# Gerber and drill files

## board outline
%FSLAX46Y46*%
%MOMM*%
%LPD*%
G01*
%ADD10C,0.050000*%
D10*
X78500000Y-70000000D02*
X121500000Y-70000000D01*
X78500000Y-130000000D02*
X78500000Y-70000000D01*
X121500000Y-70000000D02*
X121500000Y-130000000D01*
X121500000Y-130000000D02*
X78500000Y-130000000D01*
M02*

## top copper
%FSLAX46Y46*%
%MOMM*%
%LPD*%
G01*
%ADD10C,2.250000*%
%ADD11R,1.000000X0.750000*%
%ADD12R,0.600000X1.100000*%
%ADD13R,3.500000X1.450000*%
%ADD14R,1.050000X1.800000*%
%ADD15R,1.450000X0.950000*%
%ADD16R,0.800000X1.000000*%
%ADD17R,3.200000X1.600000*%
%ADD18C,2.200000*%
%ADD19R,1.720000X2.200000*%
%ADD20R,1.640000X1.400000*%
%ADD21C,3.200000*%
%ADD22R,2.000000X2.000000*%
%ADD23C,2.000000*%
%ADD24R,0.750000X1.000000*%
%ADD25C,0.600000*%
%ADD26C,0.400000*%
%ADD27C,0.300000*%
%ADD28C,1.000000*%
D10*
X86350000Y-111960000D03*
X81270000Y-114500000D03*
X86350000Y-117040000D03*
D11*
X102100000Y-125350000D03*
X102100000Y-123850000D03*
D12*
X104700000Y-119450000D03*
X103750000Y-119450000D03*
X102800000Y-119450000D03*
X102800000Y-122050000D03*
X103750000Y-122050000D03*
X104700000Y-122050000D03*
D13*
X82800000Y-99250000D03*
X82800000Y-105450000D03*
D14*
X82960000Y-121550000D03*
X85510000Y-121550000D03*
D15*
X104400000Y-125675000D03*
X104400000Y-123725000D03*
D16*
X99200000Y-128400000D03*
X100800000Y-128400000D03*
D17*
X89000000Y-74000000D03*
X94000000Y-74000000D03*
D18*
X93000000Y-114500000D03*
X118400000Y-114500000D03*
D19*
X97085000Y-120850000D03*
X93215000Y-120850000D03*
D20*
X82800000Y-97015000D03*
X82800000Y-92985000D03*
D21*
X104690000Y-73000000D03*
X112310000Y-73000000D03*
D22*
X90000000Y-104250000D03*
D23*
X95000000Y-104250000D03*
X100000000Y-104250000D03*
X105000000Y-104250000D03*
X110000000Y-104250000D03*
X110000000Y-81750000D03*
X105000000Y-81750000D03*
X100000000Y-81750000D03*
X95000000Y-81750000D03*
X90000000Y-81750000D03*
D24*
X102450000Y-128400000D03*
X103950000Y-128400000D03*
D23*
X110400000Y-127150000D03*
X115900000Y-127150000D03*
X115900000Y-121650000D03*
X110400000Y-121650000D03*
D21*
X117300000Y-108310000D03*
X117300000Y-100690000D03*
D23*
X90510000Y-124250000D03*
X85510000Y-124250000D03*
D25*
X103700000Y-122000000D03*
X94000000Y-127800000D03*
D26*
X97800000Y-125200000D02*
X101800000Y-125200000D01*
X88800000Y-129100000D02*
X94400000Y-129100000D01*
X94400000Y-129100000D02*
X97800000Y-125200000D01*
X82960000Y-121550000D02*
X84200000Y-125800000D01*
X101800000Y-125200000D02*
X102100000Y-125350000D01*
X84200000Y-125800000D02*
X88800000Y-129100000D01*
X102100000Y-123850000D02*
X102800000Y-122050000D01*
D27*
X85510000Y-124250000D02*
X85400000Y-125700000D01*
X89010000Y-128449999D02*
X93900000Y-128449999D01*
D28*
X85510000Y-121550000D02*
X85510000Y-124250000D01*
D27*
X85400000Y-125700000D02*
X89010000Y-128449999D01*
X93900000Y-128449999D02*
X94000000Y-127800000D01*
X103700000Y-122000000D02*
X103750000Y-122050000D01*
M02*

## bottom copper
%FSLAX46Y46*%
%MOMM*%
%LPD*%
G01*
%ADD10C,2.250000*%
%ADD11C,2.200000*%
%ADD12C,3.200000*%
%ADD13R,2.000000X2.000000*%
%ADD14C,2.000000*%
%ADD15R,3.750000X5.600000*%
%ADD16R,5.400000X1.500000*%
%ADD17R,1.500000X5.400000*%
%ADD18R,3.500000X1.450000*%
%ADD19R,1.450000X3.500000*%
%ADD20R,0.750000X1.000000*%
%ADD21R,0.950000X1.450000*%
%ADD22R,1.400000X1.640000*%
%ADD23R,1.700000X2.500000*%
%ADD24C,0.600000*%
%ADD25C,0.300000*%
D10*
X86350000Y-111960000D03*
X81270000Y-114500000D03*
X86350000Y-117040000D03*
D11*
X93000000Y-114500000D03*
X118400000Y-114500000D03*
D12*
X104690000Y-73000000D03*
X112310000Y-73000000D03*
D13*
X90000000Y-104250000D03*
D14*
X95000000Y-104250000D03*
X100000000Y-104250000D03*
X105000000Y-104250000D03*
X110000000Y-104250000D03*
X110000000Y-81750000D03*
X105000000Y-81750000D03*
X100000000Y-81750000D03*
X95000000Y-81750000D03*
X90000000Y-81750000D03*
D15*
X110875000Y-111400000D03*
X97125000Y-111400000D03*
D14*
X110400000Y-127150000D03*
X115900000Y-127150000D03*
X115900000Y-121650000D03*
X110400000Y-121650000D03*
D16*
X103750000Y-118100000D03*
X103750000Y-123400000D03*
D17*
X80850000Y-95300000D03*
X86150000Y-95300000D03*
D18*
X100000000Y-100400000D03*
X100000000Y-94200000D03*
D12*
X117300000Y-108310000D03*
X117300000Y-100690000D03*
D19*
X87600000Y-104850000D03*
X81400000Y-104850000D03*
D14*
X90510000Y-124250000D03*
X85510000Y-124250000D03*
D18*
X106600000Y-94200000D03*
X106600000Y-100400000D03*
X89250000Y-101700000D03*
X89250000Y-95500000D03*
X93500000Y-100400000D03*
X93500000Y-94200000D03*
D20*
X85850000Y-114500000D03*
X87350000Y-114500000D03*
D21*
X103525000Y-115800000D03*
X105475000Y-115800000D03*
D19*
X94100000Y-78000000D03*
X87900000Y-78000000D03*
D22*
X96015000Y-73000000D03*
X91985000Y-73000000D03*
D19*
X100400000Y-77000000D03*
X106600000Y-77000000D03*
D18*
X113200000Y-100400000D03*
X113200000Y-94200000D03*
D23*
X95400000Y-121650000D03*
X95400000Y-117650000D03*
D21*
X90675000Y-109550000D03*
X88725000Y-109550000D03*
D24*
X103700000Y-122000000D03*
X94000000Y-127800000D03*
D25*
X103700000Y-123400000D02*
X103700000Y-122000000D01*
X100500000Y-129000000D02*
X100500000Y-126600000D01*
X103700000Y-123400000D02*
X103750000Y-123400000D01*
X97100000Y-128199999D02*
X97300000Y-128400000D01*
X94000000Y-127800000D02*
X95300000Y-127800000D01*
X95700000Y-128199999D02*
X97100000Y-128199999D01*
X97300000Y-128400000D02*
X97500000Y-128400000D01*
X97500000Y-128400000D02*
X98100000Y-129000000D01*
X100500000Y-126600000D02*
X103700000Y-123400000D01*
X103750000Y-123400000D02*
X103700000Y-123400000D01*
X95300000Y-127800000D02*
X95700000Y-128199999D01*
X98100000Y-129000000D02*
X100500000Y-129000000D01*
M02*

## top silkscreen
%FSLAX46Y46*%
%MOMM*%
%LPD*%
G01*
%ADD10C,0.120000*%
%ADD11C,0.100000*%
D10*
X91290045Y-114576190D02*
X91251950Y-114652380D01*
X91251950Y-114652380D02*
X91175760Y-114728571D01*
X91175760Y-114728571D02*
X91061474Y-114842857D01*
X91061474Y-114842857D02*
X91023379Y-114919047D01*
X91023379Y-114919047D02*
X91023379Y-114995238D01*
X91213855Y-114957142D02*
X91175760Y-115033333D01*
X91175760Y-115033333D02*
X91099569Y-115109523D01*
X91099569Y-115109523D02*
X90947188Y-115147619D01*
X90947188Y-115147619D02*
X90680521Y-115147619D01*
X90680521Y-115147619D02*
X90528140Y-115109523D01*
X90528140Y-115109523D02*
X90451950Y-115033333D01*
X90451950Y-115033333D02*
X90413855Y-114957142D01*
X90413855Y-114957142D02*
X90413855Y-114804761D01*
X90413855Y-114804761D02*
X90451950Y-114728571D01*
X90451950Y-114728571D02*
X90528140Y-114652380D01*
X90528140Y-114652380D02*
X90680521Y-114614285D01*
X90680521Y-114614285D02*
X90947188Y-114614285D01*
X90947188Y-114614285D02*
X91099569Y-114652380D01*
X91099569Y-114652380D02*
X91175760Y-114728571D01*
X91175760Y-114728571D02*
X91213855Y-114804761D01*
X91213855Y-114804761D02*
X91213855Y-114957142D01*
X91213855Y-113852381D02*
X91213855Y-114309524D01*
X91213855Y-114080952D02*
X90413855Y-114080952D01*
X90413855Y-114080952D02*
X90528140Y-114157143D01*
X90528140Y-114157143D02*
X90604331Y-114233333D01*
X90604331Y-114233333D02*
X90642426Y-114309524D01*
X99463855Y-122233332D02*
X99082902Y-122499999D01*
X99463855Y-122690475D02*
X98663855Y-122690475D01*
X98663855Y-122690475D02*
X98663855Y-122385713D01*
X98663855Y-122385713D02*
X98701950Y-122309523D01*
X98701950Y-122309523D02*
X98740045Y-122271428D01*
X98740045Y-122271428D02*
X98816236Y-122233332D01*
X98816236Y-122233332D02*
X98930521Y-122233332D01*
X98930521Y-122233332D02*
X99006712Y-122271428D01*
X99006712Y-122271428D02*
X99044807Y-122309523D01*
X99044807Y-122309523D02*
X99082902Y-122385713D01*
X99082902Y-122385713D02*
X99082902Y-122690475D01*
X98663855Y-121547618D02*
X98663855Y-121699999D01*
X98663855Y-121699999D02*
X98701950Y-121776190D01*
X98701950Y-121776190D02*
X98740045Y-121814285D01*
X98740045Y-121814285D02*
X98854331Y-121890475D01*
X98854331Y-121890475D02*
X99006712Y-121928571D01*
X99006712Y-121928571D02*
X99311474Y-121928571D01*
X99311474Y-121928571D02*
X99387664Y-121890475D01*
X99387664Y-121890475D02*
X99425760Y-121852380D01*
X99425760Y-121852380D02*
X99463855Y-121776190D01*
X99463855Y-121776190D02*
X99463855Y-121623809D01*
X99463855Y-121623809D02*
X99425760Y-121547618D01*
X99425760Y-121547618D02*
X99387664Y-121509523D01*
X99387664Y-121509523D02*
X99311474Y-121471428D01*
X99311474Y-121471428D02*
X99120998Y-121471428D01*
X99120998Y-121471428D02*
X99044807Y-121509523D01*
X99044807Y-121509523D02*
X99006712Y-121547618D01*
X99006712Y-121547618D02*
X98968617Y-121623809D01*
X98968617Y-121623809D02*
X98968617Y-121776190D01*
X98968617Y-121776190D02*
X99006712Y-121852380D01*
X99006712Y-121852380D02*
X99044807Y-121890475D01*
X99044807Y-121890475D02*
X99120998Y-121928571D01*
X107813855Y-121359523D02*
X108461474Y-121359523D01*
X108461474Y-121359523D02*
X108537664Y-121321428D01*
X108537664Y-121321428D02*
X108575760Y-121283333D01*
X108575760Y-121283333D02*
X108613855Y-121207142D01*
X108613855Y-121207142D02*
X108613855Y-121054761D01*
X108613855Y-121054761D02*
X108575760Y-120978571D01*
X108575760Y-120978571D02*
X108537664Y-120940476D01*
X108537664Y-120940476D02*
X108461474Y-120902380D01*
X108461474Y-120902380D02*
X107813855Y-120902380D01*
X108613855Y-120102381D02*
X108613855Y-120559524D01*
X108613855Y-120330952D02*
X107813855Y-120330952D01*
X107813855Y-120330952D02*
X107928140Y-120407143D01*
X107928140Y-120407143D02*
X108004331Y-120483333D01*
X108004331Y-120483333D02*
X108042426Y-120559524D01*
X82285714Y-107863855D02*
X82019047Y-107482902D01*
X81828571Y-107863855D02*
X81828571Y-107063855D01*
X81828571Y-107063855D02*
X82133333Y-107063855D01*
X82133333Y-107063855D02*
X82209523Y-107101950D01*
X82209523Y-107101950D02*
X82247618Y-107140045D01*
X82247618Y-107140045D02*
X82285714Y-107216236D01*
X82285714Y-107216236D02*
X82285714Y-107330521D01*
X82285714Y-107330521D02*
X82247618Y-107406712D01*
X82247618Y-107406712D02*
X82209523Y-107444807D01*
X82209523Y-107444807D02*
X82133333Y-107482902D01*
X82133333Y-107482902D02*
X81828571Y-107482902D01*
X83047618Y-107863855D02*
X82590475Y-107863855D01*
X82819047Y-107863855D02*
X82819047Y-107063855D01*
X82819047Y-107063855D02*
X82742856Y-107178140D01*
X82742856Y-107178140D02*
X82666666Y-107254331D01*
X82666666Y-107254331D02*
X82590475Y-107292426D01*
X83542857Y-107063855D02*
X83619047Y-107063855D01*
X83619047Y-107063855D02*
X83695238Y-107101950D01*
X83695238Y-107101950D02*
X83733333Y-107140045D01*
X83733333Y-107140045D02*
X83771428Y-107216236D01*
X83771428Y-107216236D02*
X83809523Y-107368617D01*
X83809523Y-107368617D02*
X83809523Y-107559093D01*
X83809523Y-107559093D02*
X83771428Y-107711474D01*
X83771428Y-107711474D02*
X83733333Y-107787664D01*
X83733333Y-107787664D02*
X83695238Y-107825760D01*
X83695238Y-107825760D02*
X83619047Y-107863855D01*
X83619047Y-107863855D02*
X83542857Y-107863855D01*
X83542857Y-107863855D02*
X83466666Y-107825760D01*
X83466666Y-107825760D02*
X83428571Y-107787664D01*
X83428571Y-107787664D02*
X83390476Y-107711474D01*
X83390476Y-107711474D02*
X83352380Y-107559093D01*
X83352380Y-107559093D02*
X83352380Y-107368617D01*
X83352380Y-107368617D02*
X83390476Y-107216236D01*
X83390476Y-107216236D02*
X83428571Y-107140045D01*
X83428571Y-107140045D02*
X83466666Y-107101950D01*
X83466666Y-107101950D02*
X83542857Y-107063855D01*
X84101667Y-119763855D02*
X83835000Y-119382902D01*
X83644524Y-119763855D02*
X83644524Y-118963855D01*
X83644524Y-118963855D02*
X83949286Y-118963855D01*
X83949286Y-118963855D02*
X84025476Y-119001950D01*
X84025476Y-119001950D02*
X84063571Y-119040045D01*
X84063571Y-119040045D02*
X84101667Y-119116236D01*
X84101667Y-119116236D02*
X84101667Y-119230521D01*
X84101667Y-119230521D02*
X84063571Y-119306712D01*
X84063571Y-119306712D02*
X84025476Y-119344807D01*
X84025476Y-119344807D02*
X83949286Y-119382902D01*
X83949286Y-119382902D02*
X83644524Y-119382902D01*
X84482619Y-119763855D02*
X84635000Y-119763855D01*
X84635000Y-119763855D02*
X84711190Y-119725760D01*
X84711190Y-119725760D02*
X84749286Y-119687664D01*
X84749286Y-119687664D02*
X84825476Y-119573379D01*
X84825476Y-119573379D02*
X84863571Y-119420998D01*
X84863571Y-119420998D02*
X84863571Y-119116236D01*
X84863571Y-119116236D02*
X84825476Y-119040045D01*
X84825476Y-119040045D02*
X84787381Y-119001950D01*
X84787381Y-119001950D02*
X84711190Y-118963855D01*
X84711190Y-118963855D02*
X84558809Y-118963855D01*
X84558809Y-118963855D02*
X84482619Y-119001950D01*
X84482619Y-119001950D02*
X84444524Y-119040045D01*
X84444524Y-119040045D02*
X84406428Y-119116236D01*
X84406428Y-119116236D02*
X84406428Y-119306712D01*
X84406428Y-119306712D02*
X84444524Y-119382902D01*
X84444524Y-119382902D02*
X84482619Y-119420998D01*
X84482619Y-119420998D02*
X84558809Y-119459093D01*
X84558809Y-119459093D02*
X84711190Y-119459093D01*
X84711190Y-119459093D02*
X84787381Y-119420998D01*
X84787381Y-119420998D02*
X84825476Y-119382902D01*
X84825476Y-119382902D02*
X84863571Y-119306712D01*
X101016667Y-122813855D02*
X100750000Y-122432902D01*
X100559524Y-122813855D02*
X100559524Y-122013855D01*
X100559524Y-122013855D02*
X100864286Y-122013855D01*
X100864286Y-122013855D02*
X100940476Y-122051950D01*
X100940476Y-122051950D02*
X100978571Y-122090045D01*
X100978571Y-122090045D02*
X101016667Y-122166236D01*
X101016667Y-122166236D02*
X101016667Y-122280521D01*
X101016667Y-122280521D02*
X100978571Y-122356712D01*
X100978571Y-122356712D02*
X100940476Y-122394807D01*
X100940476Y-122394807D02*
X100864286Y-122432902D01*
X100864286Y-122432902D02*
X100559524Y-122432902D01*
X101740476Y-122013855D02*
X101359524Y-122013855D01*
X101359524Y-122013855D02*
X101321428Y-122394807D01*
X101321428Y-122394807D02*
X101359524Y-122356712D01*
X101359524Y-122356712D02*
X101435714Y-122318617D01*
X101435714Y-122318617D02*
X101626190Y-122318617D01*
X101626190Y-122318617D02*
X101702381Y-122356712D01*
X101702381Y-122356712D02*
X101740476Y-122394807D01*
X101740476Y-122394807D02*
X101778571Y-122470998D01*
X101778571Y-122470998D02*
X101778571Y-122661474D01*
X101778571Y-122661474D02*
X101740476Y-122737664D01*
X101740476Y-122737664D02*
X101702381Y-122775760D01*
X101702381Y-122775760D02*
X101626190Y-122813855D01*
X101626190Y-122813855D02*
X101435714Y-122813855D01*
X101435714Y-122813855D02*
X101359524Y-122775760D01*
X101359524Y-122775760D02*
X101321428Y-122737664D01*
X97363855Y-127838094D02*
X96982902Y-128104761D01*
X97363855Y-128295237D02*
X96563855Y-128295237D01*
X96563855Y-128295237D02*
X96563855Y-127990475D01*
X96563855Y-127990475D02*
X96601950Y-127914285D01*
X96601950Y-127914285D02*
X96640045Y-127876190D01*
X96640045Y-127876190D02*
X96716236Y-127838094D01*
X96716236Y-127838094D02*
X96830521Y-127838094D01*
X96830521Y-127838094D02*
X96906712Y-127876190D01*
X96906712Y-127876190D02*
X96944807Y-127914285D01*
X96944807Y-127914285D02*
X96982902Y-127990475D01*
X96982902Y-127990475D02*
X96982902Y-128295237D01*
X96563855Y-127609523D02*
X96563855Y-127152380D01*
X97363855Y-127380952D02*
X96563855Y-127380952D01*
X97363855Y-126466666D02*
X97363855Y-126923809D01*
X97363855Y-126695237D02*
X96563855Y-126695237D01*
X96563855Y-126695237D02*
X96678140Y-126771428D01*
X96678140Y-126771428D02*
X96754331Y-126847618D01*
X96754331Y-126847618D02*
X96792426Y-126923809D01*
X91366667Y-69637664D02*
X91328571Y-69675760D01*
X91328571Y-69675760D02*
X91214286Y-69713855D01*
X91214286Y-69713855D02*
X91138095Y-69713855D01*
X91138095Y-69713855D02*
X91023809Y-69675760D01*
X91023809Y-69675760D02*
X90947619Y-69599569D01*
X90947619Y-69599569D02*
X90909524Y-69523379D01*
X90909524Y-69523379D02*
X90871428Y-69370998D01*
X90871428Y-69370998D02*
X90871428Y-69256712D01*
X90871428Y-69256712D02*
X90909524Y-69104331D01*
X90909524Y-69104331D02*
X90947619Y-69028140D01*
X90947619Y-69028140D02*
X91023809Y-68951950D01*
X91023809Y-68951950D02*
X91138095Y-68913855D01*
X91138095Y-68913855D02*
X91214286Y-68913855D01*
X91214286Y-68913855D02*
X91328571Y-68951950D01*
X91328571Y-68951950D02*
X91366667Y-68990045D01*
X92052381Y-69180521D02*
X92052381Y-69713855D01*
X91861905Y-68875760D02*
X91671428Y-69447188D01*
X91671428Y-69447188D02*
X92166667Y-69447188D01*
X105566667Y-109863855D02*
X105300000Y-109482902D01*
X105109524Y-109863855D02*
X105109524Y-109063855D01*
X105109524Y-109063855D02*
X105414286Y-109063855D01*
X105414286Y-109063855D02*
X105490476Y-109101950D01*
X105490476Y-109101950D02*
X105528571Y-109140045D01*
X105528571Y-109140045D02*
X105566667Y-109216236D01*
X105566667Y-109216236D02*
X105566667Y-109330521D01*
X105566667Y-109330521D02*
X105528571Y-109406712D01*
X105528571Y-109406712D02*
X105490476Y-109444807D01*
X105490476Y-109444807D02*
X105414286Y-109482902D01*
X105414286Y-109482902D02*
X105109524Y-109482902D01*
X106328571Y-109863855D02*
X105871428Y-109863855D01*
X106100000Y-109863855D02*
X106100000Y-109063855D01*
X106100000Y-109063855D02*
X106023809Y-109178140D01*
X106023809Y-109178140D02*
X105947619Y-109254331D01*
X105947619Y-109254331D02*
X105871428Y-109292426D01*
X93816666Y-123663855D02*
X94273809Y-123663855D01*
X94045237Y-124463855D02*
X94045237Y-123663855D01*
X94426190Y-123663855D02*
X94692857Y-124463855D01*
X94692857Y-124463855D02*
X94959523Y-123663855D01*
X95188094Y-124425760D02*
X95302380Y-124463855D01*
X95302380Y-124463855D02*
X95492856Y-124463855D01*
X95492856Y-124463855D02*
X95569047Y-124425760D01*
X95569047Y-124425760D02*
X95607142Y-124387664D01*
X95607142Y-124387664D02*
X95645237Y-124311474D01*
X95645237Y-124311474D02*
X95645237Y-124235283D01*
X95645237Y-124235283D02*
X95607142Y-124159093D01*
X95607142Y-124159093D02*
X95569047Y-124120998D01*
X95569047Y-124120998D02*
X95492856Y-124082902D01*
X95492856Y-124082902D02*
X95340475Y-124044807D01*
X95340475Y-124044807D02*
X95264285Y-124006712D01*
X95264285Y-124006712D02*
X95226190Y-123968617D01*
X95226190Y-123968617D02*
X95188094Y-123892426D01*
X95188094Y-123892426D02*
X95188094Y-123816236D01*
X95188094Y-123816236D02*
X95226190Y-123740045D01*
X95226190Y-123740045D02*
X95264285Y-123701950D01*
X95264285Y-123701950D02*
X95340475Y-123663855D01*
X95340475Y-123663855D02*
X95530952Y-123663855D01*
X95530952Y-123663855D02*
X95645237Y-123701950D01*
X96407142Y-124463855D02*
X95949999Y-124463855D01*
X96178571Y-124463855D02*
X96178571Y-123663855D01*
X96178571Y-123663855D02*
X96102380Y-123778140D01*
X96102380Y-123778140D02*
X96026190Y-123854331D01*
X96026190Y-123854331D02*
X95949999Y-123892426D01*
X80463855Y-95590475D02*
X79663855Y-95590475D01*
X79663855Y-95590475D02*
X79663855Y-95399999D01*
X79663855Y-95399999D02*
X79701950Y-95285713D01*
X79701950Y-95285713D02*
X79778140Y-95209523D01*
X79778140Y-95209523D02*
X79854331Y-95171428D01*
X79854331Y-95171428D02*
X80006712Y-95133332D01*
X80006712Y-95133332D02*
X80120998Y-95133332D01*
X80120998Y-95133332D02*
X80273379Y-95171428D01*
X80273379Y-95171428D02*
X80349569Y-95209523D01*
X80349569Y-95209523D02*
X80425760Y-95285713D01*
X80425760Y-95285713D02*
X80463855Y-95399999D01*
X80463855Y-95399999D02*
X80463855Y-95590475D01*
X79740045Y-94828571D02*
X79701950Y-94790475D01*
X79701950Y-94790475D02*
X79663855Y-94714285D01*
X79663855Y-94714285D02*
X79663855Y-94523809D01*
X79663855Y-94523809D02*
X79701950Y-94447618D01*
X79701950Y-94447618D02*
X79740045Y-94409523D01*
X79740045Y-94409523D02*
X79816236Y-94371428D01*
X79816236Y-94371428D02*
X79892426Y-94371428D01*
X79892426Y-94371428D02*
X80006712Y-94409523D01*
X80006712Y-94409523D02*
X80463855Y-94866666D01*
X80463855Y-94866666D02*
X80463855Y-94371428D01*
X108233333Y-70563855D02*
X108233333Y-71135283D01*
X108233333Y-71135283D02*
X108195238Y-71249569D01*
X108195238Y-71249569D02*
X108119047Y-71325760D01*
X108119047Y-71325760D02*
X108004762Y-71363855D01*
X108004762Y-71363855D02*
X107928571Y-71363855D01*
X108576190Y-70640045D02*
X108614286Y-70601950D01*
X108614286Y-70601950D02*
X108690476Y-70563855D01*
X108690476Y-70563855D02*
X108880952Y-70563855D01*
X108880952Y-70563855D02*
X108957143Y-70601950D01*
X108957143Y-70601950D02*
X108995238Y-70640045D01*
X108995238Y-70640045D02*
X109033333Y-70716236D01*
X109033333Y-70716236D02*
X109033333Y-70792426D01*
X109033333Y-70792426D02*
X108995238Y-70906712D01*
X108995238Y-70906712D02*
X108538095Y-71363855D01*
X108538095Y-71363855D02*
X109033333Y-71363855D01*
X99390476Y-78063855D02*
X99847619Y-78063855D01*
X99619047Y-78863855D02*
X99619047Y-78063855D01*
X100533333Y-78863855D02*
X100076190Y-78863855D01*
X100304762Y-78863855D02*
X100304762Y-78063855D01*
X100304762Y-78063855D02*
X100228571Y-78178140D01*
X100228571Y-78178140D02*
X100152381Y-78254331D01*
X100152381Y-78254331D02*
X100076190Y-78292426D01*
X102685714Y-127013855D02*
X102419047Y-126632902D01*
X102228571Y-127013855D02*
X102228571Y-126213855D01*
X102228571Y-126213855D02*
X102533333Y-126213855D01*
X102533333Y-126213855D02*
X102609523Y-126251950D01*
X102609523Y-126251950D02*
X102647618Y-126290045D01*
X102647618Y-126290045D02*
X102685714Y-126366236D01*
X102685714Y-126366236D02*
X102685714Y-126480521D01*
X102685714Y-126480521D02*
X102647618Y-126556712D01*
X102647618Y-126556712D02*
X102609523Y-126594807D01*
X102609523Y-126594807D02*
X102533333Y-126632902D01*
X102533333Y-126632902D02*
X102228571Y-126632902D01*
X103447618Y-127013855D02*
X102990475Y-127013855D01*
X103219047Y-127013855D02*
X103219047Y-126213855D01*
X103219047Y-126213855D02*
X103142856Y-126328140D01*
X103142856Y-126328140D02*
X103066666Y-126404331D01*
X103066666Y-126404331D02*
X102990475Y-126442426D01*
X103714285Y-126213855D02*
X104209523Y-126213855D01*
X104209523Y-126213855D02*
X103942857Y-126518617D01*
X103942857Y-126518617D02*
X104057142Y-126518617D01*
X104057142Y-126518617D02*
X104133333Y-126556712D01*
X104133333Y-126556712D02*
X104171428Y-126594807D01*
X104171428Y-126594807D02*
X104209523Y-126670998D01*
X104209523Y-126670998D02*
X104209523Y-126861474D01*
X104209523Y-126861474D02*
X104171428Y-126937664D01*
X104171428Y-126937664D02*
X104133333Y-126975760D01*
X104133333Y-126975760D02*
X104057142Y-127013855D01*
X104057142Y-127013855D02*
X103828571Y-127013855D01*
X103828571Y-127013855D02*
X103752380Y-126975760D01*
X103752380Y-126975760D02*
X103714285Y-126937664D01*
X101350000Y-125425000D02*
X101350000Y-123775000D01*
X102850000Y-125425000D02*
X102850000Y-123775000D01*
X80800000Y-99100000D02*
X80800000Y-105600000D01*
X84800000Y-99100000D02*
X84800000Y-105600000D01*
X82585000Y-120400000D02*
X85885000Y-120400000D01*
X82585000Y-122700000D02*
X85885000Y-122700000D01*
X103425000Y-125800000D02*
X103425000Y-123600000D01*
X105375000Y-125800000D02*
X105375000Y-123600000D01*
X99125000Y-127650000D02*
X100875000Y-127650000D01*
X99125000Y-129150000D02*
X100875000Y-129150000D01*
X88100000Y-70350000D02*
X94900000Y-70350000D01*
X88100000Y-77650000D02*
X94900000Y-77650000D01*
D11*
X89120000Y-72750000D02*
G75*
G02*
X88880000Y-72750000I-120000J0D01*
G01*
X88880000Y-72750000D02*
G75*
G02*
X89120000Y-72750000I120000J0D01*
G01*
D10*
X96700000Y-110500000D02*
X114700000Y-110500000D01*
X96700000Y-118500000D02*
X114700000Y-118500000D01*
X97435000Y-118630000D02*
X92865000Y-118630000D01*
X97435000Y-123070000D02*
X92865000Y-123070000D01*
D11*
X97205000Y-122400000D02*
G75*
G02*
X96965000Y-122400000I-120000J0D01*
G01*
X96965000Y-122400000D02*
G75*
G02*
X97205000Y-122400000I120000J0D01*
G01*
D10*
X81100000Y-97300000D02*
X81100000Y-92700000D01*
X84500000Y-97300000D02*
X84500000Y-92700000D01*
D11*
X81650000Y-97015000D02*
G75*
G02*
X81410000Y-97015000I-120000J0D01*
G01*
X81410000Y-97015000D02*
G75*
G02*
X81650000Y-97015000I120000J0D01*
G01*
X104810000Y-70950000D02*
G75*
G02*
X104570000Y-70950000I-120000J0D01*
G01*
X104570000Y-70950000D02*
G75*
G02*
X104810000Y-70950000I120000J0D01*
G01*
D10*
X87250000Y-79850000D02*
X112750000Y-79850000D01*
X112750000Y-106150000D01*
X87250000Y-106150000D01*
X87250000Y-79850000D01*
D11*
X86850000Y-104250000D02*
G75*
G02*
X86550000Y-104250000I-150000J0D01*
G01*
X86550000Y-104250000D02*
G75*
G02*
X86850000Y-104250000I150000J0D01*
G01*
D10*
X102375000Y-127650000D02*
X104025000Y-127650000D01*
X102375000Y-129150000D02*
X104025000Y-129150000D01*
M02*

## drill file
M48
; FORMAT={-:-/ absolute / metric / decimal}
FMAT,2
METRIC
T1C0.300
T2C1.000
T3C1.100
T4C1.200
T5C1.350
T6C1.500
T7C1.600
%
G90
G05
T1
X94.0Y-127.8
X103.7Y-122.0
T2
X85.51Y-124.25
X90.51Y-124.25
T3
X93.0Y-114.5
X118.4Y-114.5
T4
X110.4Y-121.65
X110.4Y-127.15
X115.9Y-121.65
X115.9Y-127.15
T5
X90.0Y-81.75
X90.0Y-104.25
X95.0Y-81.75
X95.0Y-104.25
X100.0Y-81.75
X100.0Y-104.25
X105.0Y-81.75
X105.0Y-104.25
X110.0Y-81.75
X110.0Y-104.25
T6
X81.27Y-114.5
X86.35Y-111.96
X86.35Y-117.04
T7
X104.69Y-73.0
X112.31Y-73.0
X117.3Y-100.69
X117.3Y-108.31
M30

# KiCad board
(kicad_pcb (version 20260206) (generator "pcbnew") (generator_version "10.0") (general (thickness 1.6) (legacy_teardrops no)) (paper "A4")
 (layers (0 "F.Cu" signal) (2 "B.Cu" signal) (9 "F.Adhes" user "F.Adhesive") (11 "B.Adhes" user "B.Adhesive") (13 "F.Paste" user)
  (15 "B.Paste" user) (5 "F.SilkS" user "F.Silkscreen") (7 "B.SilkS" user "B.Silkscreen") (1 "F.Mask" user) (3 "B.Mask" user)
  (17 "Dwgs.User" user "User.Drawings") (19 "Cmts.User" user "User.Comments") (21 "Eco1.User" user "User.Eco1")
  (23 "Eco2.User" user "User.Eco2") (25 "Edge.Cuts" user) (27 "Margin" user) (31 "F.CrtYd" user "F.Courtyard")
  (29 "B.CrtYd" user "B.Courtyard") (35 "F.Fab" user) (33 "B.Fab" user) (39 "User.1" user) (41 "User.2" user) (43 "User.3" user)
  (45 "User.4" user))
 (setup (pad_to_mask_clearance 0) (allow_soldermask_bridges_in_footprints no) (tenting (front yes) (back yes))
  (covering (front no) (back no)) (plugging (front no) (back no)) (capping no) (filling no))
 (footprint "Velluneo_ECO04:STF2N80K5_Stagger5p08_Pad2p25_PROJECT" (layer "F.Cu") (at 86.35 114.5 -90)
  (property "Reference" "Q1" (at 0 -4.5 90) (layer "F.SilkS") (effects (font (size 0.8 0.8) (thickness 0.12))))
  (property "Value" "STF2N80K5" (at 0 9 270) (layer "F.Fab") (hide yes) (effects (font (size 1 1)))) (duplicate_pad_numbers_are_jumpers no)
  (pad "1" thru_hole circle (at -2.54 0 270) (size 2.25 2.25) (drill 1.5) (layers "*.Cu" "*.Mask") (remove_unused_layers no) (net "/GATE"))
  (pad "2" thru_hole circle (at 0 5.08 270) (size 2.25 2.25) (drill 1.5) (layers "*.Cu" "*.Mask") (remove_unused_layers no) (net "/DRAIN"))
  (pad "3" thru_hole circle (at 2.54 0 270) (size 2.25 2.25) (drill 1.5) (layers "*.Cu" "*.Mask") (remove_unused_layers no) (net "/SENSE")))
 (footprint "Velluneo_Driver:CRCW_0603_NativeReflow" (layer "F.Cu") (at 102.1 124.6 90)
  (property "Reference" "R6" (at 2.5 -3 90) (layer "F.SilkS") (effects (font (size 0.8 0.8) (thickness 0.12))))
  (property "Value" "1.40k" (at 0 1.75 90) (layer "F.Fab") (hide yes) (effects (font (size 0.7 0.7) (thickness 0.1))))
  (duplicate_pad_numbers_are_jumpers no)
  (fp_line (start -0.825 -0.75) (end 0.825 -0.75) (stroke (width 0.12) (type default)) (layer "F.SilkS"))
  (fp_line (start -0.825 0.75) (end 0.825 0.75) (stroke (width 0.12) (type default)) (layer "F.SilkS"))
  (pad "1" smd rect (at -0.75 0 90) (size 0.75 1) (layers "F.Cu" "F.Mask" "F.Paste") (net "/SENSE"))
  (pad "2" smd rect (at 0.75 0 90) (size 0.75 1) (layers "F.Cu" "F.Mask" "F.Paste") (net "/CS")))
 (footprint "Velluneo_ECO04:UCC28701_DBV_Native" (layer "F.Cu") (at 103.75 120.75 -90)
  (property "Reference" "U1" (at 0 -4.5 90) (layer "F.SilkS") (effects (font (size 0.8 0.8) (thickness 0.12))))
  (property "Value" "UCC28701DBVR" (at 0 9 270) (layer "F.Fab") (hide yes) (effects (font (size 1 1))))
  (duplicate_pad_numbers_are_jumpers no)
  (pad "1" smd rect (at -1.3 -0.95 270) (size 1.1 0.6) (layers "F.Cu" "F.Mask" "F.Paste") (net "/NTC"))
  (pad "2" smd rect (at -1.3 0 270) (size 1.1 0.6) (layers "F.Cu" "F.Mask" "F.Paste") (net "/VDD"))
  (pad "3" smd rect (at -1.3 0.95 270) (size 1.1 0.6) (layers "F.Cu" "F.Mask" "F.Paste") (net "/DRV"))
  (pad "4" smd rect (at 1.3 0.95 270) (size 1.1 0.6) (layers "F.Cu" "F.Mask" "F.Paste") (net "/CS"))
  (pad "5" smd rect (at 1.3 0 270) (size 1.1 0.6) (layers "F.Cu" "F.Mask" "F.Paste") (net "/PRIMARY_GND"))
  (pad "6" smd rect (at 1.3 -0.95 270) (size 1.1 0.6) (layers "F.Cu" "F.Mask" "F.Paste") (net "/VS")))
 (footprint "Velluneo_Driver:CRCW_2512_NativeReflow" (layer "F.Cu") (at 82.8 102.35 -90)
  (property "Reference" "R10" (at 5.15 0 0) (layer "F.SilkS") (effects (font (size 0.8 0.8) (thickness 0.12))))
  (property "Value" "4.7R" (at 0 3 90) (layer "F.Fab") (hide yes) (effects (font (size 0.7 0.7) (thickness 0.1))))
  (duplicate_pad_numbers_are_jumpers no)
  (fp_line (start -3.25 2) (end 3.25 2) (stroke (width 0.12) (type default)) (layer "F.SilkS"))
  (fp_line (start -3.25 -2) (end 3.25 -2) (stroke (width 0.12) (type default)) (layer "F.SilkS"))
  (pad "1" smd rect (at -3.1 0 270) (size 1.45 3.5) (layers "F.Cu" "F.Mask" "F.Paste") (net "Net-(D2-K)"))
  (pad "2" smd rect (at 3.1 0 270) (size 1.45 3.5) (layers "F.Cu" "F.Mask" "F.Paste") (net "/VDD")))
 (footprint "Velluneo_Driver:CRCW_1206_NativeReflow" (layer "F.Cu") (at 84.235 121.55)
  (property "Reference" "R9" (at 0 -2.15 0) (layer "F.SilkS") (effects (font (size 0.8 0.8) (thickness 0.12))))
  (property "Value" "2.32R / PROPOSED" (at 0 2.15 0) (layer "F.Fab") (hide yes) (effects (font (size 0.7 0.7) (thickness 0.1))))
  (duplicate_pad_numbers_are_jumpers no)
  (fp_line (start -1.65 -1.15) (end 1.65 -1.15) (stroke (width 0.12) (type default)) (layer "F.SilkS"))
  (fp_line (start -1.65 1.15) (end 1.65 1.15) (stroke (width 0.12) (type default)) (layer "F.SilkS"))
  (pad "1" smd rect (at -1.275 0) (size 1.05 1.8) (layers "F.Cu" "F.Mask" "F.Paste") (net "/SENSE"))
  (pad "2" smd rect (at 1.275 0) (size 1.05 1.8) (layers "F.Cu" "F.Mask" "F.Paste") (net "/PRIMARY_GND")))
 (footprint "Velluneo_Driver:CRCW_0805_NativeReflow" (layer "F.Cu") (at 104.4 124.7 90)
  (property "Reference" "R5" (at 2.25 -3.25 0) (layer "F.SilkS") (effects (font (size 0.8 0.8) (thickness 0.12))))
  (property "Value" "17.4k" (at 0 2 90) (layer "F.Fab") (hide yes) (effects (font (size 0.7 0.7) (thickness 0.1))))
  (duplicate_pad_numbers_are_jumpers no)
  (fp_line (start -1.1 -0.975) (end 1.1 -0.975) (stroke (width 0.12) (type default)) (layer "F.SilkS"))
  (fp_line (start -1.1 0.975) (end 1.1 0.975) (stroke (width 0.12) (type default)) (layer "F.SilkS"))
  (pad "1" smd rect (at -0.975 0 90) (size 0.95 1.45) (layers "F.Cu" "F.Mask" "F.Paste") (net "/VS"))
  (pad "2" smd rect (at 0.975 0 90) (size 0.95 1.45) (layers "F.Cu" "F.Mask" "F.Paste") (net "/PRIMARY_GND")))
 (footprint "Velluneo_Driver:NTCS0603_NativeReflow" (layer "F.Cu") (at 100 128.4)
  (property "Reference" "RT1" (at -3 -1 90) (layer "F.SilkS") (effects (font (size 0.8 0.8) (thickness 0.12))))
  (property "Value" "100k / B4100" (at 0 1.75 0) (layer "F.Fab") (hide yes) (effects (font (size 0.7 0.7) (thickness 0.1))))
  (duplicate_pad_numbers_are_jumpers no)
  (fp_line (start -0.875 -0.75) (end 0.875 -0.75) (stroke (width 0.12) (type default)) (layer "F.SilkS"))
  (fp_line (start -0.875 0.75) (end 0.875 0.75) (stroke (width 0.12) (type default)) (layer "F.SilkS"))
  (pad "1" smd rect (at -0.8 0) (size 0.8 1) (layers "F.Cu" "F.Mask" "F.Paste") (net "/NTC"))
  (pad "2" smd rect (at 0.8 0) (size 0.8 1) (layers "F.Cu" "F.Mask" "F.Paste") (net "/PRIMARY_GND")))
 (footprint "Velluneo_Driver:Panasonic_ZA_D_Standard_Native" (layer "F.Cu") (at 91.5 74)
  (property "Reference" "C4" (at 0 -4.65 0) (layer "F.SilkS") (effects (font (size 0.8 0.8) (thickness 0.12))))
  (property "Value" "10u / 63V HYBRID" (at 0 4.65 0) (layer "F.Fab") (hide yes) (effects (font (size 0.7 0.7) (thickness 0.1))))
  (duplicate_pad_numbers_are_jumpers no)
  (fp_line (start -3.4 -3.65) (end 3.4 -3.65) (stroke (width 0.12) (type default)) (layer "F.SilkS"))
  (fp_line (start -3.4 3.65) (end 3.4 3.65) (stroke (width 0.12) (type default)) (layer "F.SilkS"))
  (fp_circle (center -2.5 -1.25) (end -2.38 -1.25) (stroke (width 0.1) (type default)) (fill no) (layer "F.SilkS"))
  (pad "1" smd rect (at -2.5 0) (size 3.2 1.6) (layers "F.Cu" "F.Mask" "F.Paste") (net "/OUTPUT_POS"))
  (pad "2" smd rect (at 2.5 0) (size 3.2 1.6) (layers "F.Cu" "F.Mask" "F.Paste") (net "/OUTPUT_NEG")))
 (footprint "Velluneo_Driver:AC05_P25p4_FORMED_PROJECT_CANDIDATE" (layer "F.Cu") (at 105.7 114.5)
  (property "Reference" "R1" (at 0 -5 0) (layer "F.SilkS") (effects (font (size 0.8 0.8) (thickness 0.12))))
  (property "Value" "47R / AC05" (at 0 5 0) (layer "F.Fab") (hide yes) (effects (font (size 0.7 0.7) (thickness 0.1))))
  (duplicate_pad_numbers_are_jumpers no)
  (fp_line (start -9 -4) (end 9 -4) (stroke (width 0.12) (type default)) (layer "F.SilkS"))
  (fp_line (start -9 4) (end 9 4) (stroke (width 0.12) (type default)) (layer "F.SilkS"))
  (pad "1" thru_hole circle (at -12.7 0) (size 2.2 2.2) (drill 1.1) (layers "*.Cu" "*.Mask") (remove_unused_layers no) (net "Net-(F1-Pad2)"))
  (pad "2" thru_hole circle (at 12.7 0) (size 2.2 2.2) (drill 1.1) (layers "*.Cu" "*.Mask") (remove_unused_layers no)
   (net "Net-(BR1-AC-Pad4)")))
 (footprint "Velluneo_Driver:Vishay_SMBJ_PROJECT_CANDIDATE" (layer "F.Cu") (at 95.15 120.85 180)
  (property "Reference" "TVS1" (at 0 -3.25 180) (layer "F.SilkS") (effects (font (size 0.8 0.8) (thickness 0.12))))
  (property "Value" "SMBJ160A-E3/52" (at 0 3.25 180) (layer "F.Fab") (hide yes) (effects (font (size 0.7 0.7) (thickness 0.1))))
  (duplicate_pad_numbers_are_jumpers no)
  (fp_line (start -2.285 2.22) (end 2.285 2.22) (stroke (width 0.12) (type default)) (layer "F.SilkS"))
  (fp_line (start -2.285 -2.22) (end 2.285 -2.22) (stroke (width 0.12) (type default)) (layer "F.SilkS"))
  (fp_circle (center -1.935 -1.55) (end -1.815 -1.55) (stroke (width 0.1) (type default)) (fill no) (layer "F.SilkS"))
  (pad "1" smd rect (at -1.935 0 180) (size 1.72 2.2) (layers "F.Cu" "F.Mask" "F.Paste") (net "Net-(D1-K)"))
  (pad "2" smd rect (at 1.935 0 180) (size 1.72 2.2) (layers "F.Cu" "F.Mask" "F.Paste") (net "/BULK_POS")))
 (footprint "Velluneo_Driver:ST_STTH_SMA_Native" (layer "F.Cu") (at 82.8 95 90)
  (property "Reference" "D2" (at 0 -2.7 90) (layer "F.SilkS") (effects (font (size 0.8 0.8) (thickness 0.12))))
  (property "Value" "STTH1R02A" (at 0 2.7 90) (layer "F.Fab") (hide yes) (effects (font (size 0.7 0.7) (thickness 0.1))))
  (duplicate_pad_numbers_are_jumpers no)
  (fp_line (start -2.3 -1.7) (end 2.3 -1.7) (stroke (width 0.12) (type default)) (layer "F.SilkS"))
  (fp_line (start -2.3 1.7) (end 2.3 1.7) (stroke (width 0.12) (type default)) (layer "F.SilkS"))
  (fp_circle (center -2.015 -1.27) (end -1.895 -1.27) (stroke (width 0.1) (type default)) (fill no) (layer "F.SilkS"))
  (pad "1" smd rect (at -2.015 0 90) (size 1.4 1.64) (layers "F.Cu" "F.Mask" "F.Paste") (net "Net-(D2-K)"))
  (pad "2" smd rect (at 2.015 0 90) (size 1.4 1.64) (layers "F.Cu" "F.Mask" "F.Paste") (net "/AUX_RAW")))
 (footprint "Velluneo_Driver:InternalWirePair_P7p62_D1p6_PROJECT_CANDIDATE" (layer "F.Cu") (at 108.5 73)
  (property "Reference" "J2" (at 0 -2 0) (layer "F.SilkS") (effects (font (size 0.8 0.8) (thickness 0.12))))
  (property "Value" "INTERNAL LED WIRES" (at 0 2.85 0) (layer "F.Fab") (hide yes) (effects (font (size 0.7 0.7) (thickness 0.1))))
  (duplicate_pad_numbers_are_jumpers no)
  (fp_circle (center -3.81 -2.05) (end -3.69 -2.05) (stroke (width 0.1) (type default)) (fill no) (layer "F.SilkS"))
  (pad "1" thru_hole circle (at -3.81 0) (size 3.2 3.2) (drill 1.6) (layers "*.Cu" "*.Mask") (remove_unused_layers no) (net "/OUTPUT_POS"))
  (pad "2" thru_hole circle (at 3.81 0) (size 3.2 3.2) (drill 1.6) (layers "*.Cu" "*.Mask") (remove_unused_layers no) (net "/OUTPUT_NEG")))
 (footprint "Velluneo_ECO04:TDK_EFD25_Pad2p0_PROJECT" (layer "F.Cu") (at 100 93)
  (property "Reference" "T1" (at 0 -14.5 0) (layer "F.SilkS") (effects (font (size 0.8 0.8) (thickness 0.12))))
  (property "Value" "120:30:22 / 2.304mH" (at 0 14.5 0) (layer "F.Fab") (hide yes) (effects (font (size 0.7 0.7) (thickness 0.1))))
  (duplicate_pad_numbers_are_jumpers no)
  (fp_rect (start -12.75 -13.15) (end 12.75 13.15) (stroke (width 0.12) (type default)) (fill no) (layer "F.SilkS"))
  (fp_circle (center -13.3 11.25) (end -13.15 11.25) (stroke (width 0.1) (type default)) (fill no) (layer "F.SilkS"))
  (pad "1" thru_hole rect (at -10 11.25) (size 2 2) (drill 1.35) (layers "*.Cu" "*.Mask") (remove_unused_layers no) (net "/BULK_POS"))
  (pad "2" thru_hole circle (at -5 11.25) (size 2 2) (drill 1.35) (layers "*.Cu" "*.Mask") (remove_unused_layers no) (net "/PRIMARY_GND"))
  (pad "3" thru_hole circle (at 0 11.25) (size 2 2) (drill 1.35) (layers "*.Cu" "*.Mask") (remove_unused_layers no)
   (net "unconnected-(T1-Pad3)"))
  (pad "4" thru_hole circle (at 5 11.25) (size 2 2) (drill 1.35) (layers "*.Cu" "*.Mask") (remove_unused_layers no) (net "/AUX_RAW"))
  (pad "5" thru_hole circle (at 10 11.25) (size 2 2) (drill 1.35) (layers "*.Cu" "*.Mask") (remove_unused_layers no) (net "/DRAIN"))
  (pad "6" thru_hole circle (at 10 -11.25) (size 2 2) (drill 1.35) (layers "*.Cu" "*.Mask") (remove_unused_layers no) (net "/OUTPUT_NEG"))
  (pad "7" thru_hole circle (at 5 -11.25) (size 2 2) (drill 1.35) (layers "*.Cu" "*.Mask") (remove_unused_layers no)
   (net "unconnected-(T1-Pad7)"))
  (pad "8" thru_hole circle (at 0 -11.25) (size 2 2) (drill 1.35) (layers "*.Cu" "*.Mask") (remove_unused_layers no)
   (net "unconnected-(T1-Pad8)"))
  (pad "9" thru_hole circle (at -5 -11.25) (size 2 2) (drill 1.35) (layers "*.Cu" "*.Mask") (remove_unused_layers no)
   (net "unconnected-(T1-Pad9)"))
  (pad "10" thru_hole circle (at -10 -11.25) (size 2 2) (drill 1.35) (layers "*.Cu" "*.Mask") (remove_unused_layers no)
   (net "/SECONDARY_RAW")))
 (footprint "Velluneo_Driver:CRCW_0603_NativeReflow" (layer "F.Cu") (at 103.2 128.4)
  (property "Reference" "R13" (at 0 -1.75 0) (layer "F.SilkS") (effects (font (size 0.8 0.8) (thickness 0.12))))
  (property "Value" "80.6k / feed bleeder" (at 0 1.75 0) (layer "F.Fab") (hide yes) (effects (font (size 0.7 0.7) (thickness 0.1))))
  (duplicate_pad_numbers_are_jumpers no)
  (fp_line (start -0.825 -0.75) (end 0.825 -0.75) (stroke (width 0.12) (type default)) (layer "F.SilkS"))
  (fp_line (start -0.825 0.75) (end 0.825 0.75) (stroke (width 0.12) (type default)) (layer "F.SilkS"))
  (pad "1" smd rect (at -0.75 0) (size 0.75 1) (layers "F.Cu" "F.Mask" "F.Paste") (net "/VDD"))
  (pad "2" smd rect (at 0.75 0) (size 0.75 1) (layers "F.Cu" "F.Mask" "F.Paste") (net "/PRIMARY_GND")))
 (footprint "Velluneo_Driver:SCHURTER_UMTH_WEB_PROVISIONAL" (layer "B.Cu") (at 104 111.4 180)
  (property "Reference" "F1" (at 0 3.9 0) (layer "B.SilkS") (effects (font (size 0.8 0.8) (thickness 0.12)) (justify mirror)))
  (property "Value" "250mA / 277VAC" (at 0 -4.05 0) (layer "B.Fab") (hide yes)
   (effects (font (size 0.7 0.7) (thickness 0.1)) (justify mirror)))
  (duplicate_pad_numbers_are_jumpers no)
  (pad "1" smd rect (at -6.875 0 180) (size 3.75 5.6) (layers "B.Cu" "B.Mask" "B.Paste") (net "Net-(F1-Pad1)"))
  (pad "2" smd rect (at 6.875 0 180) (size 3.75 5.6) (layers "B.Cu" "B.Mask" "B.Paste") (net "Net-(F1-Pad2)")))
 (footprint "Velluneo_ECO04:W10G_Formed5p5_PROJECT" (layer "B.Cu") (at 113.15 124.4)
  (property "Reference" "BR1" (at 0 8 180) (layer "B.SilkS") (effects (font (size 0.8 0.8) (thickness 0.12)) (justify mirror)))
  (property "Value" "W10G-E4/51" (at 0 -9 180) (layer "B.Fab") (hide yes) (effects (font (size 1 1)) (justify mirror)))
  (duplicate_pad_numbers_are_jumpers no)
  (pad "1" thru_hole circle (at -2.75 2.75) (size 2 2) (drill 1.2) (layers "*.Cu" "*.Mask") (remove_unused_layers no) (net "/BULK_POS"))
  (pad "2" thru_hole circle (at 2.75 2.75) (size 2 2) (drill 1.2) (layers "*.Cu" "*.Mask") (remove_unused_layers no)
   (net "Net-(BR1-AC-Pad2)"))
  (pad "3" thru_hole circle (at 2.75 -2.75) (size 2 2) (drill 1.2) (layers "*.Cu" "*.Mask") (remove_unused_layers no) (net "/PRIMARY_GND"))
  (pad "4" thru_hole circle (at -2.75 -2.75) (size 2 2) (drill 1.2) (layers "*.Cu" "*.Mask") (remove_unused_layers no)
   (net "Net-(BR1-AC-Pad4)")))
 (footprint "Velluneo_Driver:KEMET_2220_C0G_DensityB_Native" (layer "B.Cu") (at 103.75 120.75 -90)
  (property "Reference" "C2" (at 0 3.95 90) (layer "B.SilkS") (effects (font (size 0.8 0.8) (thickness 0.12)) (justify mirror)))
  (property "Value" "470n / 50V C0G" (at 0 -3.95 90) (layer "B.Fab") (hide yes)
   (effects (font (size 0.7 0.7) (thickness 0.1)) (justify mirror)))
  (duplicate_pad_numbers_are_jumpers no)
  (pad "1" smd rect (at -2.65 0 270) (size 1.5 5.4) (layers "B.Cu" "B.Mask" "B.Paste") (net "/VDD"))
  (pad "2" smd rect (at 2.65 0 270) (size 1.5 5.4) (layers "B.Cu" "B.Mask" "B.Paste") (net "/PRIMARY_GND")))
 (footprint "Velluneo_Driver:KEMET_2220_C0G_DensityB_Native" (layer "B.Cu") (at 83.5 95.3)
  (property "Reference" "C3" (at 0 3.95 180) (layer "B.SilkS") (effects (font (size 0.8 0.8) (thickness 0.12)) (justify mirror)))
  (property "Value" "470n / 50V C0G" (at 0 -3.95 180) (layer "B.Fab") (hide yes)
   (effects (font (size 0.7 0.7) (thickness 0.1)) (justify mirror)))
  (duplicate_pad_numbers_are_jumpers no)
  (pad "1" smd rect (at -2.65 0) (size 1.5 5.4) (layers "B.Cu" "B.Mask" "B.Paste") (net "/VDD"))
  (pad "2" smd rect (at 2.65 0) (size 1.5 5.4) (layers "B.Cu" "B.Mask" "B.Paste") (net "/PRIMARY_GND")))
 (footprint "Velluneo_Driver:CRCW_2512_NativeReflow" (layer "B.Cu") (at 100 97.3 90)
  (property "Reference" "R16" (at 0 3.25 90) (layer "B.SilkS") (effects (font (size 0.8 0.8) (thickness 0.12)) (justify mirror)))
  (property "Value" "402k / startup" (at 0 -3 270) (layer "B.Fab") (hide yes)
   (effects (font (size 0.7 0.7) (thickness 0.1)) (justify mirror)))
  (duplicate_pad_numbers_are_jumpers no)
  (pad "1" smd rect (at -3.1 0 90) (size 1.45 3.5) (layers "B.Cu" "B.Mask" "B.Paste") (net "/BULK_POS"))
  (pad "2" smd rect (at 3.1 0 90) (size 1.45 3.5) (layers "B.Cu" "B.Mask" "B.Paste") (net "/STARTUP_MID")))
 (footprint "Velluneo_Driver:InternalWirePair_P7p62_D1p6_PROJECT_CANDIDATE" (layer "B.Cu") (at 117.3 104.5 90)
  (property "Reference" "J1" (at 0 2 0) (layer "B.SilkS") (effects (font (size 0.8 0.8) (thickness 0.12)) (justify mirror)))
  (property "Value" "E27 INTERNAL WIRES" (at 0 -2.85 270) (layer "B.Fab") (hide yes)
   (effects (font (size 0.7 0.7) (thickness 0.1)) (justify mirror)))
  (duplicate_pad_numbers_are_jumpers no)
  (pad "1" thru_hole circle (at -3.81 0 90) (size 3.2 3.2) (drill 1.6) (layers "*.Cu" "*.Mask") (remove_unused_layers no)
   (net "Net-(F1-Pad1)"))
  (pad "2" thru_hole circle (at 3.81 0 90) (size 3.2 3.2) (drill 1.6) (layers "*.Cu" "*.Mask") (remove_unused_layers no)
   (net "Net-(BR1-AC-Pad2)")))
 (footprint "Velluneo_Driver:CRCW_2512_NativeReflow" (layer "B.Cu") (at 84.5 104.85 180)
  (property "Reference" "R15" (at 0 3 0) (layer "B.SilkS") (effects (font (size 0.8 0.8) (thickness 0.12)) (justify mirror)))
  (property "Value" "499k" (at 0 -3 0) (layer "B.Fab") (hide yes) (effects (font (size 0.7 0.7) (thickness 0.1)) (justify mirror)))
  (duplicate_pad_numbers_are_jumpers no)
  (pad "1" smd rect (at -3.1 0 180) (size 1.45 3.5) (layers "B.Cu" "B.Mask" "B.Paste") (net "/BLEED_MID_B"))
  (pad "2" smd rect (at 3.1 0 180) (size 1.45 3.5) (layers "B.Cu" "B.Mask" "B.Paste") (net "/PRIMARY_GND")))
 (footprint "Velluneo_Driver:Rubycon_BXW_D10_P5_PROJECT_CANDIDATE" (layer "B.Cu") (at 88.01 124.25 180)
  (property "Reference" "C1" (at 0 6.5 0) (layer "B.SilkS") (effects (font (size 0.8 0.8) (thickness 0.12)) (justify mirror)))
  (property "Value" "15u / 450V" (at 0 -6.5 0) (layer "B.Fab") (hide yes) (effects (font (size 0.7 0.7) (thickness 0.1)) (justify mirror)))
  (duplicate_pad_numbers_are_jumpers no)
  (pad "1" thru_hole circle (at -2.5 0 180) (size 2 2) (drill 1) (layers "*.Cu" "*.Mask") (remove_unused_layers no) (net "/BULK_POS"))
  (pad "2" thru_hole circle (at 2.5 0 180) (size 2 2) (drill 1) (layers "*.Cu" "*.Mask") (remove_unused_layers no) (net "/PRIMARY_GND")))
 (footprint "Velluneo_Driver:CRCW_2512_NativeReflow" (layer "B.Cu") (at 106.6 97.3 -90)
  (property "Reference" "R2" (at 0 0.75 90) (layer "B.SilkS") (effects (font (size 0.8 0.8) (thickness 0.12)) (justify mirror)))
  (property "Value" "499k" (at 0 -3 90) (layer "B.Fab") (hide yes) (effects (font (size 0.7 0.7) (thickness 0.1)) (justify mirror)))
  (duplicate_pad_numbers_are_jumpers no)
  (pad "1" smd rect (at -3.1 0 270) (size 1.45 3.5) (layers "B.Cu" "B.Mask" "B.Paste") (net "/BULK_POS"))
  (pad "2" smd rect (at 3.1 0 270) (size 1.45 3.5) (layers "B.Cu" "B.Mask" "B.Paste") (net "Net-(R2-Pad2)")))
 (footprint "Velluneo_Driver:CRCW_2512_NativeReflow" (layer "B.Cu") (at 89.25 98.6 90)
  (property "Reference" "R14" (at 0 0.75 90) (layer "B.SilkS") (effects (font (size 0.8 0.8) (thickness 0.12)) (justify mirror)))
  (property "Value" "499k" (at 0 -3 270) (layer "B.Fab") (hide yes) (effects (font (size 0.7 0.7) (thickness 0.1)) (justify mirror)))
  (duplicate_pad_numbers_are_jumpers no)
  (pad "1" smd rect (at -3.1 0 90) (size 1.45 3.5) (layers "B.Cu" "B.Mask" "B.Paste") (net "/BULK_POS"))
  (pad "2" smd rect (at 3.1 0 90) (size 1.45 3.5) (layers "B.Cu" "B.Mask" "B.Paste") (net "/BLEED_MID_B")))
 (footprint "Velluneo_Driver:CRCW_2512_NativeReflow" (layer "B.Cu") (at 93.5 97.3 90)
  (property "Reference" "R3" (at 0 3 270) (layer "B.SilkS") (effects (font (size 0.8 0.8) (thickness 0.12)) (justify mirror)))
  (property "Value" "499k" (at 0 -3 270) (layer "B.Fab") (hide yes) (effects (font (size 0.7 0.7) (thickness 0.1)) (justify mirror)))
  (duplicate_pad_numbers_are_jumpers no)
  (pad "1" smd rect (at -3.1 0 90) (size 1.45 3.5) (layers "B.Cu" "B.Mask" "B.Paste") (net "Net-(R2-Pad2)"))
  (pad "2" smd rect (at 3.1 0 90) (size 1.45 3.5) (layers "B.Cu" "B.Mask" "B.Paste") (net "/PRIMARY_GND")))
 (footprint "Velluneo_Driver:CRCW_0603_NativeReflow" (layer "B.Cu") (at 86.6 114.5)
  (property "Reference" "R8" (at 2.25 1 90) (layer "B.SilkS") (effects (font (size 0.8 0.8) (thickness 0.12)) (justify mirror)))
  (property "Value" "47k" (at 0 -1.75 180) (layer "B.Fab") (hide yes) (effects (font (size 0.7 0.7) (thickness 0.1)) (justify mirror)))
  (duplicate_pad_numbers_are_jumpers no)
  (pad "1" smd rect (at -0.75 0) (size 0.75 1) (layers "B.Cu" "B.Mask" "B.Paste") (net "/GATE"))
  (pad "2" smd rect (at 0.75 0) (size 0.75 1) (layers "B.Cu" "B.Mask" "B.Paste") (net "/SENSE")))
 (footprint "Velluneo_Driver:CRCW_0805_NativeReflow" (layer "B.Cu") (at 104.5 115.8)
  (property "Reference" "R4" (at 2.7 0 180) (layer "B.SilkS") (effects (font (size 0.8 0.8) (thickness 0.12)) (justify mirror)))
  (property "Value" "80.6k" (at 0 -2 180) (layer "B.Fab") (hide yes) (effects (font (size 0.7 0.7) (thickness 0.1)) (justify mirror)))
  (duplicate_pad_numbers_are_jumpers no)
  (pad "1" smd rect (at -0.975 0) (size 0.95 1.45) (layers "B.Cu" "B.Mask" "B.Paste") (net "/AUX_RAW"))
  (pad "2" smd rect (at 0.975 0) (size 0.95 1.45) (layers "B.Cu" "B.Mask" "B.Paste") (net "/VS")))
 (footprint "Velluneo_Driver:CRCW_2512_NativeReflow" (layer "B.Cu") (at 91 78 180)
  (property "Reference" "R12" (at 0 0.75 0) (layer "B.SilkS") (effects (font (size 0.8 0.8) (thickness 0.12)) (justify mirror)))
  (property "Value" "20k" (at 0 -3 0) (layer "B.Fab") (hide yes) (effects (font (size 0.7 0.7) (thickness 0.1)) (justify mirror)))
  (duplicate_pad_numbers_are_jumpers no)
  (pad "1" smd rect (at -3.1 0 180) (size 1.45 3.5) (layers "B.Cu" "B.Mask" "B.Paste") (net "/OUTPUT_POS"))
  (pad "2" smd rect (at 3.1 0 180) (size 1.45 3.5) (layers "B.Cu" "B.Mask" "B.Paste") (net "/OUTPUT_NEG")))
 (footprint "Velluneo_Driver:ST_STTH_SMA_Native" (layer "B.Cu") (at 94 73 180)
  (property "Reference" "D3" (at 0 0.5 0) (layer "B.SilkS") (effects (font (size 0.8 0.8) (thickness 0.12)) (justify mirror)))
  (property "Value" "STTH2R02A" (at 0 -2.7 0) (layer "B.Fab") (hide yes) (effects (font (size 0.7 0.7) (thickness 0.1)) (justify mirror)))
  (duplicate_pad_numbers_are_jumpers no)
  (pad "1" smd rect (at -2.015 0 180) (size 1.4 1.64) (layers "B.Cu" "B.Mask" "B.Paste") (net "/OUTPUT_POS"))
  (pad "2" smd rect (at 2.015 0 180) (size 1.4 1.64) (layers "B.Cu" "B.Mask" "B.Paste") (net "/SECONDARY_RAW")))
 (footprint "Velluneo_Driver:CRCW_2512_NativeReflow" (layer "B.Cu") (at 103.5 77)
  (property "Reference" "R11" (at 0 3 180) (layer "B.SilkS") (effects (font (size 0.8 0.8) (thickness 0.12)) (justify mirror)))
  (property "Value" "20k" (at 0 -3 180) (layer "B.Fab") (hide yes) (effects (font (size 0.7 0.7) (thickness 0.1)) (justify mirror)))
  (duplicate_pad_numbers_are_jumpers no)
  (pad "1" smd rect (at -3.1 0) (size 1.45 3.5) (layers "B.Cu" "B.Mask" "B.Paste") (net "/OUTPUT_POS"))
  (pad "2" smd rect (at 3.1 0) (size 1.45 3.5) (layers "B.Cu" "B.Mask" "B.Paste") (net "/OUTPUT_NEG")))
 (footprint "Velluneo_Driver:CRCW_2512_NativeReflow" (layer "B.Cu") (at 113.2 97.3 90)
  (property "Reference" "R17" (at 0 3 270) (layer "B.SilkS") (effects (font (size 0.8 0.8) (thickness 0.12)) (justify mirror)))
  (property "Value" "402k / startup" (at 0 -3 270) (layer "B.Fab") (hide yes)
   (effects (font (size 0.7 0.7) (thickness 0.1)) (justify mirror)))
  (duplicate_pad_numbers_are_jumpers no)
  (pad "1" smd rect (at -3.1 0 90) (size 1.45 3.5) (layers "B.Cu" "B.Mask" "B.Paste") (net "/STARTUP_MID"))
  (pad "2" smd rect (at 3.1 0 90) (size 1.45 3.5) (layers "B.Cu" "B.Mask" "B.Paste") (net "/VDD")))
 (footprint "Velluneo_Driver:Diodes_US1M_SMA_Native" (layer "B.Cu") (at 95.4 119.65 90)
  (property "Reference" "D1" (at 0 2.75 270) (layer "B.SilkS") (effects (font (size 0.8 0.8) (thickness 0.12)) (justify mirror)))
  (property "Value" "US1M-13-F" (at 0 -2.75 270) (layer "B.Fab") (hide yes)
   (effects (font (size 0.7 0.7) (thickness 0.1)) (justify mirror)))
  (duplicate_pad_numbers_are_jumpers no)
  (pad "1" smd rect (at -2 0 90) (size 2.5 1.7) (layers "B.Cu" "B.Mask" "B.Paste") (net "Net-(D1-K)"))
  (pad "2" smd rect (at 2 0 90) (size 2.5 1.7) (layers "B.Cu" "B.Mask" "B.Paste") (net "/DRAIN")))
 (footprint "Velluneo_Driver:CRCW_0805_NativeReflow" (layer "B.Cu") (at 89.7 109.55 180)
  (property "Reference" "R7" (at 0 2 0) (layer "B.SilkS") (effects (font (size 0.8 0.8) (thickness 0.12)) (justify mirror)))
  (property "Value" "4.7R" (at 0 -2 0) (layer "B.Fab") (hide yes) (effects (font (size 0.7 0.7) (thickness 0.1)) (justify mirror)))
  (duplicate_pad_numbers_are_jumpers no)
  (pad "1" smd rect (at -0.975 0 180) (size 0.95 1.45) (layers "B.Cu" "B.Mask" "B.Paste") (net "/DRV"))
  (pad "2" smd rect (at 0.975 0 180) (size 0.95 1.45) (layers "B.Cu" "B.Mask" "B.Paste") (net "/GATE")))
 (gr_line (start 78.5 70) (end 121.5 70) (stroke (width 0.05) (type default)) (layer "Edge.Cuts"))
 (gr_line (start 78.5 130) (end 78.5 70) (stroke (width 0.05) (type default)) (layer "Edge.Cuts"))
 (gr_line (start 121.5 70) (end 121.5 130) (stroke (width 0.05) (type default)) (layer "Edge.Cuts"))
 (gr_line (start 121.5 130) (end 78.5 130) (stroke (width 0.05) (type default)) (layer "Edge.Cuts"))
 (segment (start 97.8 125.2) (end 101.8 125.2) (width 0.4) (layer "F.Cu") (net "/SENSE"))
 (segment (start 88.8 129.1) (end 94.4 129.1) (width 0.4) (layer "F.Cu") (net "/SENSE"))
 (segment (start 94.4 129.1) (end 97.8 125.2) (width 0.4) (layer "F.Cu") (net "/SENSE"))
 (segment (start 82.96 121.55) (end 84.2 125.8) (width 0.4) (layer "F.Cu") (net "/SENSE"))
 (segment (start 101.8 125.2) (end 102.1 125.35) (width 0.4) (layer "F.Cu") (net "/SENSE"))
 (segment (start 84.2 125.8) (end 88.8 129.1) (width 0.4) (layer "F.Cu") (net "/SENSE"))
 (segment (start 102.1 123.85) (end 102.8 122.05) (width 0.4) (layer "F.Cu") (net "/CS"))
 (segment (start 85.51 124.25) (end 85.4 125.7) (width 0.3) (layer "F.Cu") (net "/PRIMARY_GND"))
 (segment (start 89.01 128.449999) (end 93.9 128.449999) (width 0.3) (layer "F.Cu") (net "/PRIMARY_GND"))
 (segment (start 85.51 121.55) (end 85.51 124.25) (width 1) (layer "F.Cu") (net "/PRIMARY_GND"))
 (segment (start 85.4 125.7) (end 89.01 128.449999) (width 0.3) (layer "F.Cu") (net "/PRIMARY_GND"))
 (segment (start 93.9 128.449999) (end 94 127.8) (width 0.3) (layer "F.Cu") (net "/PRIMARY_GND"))
 (segment (start 103.7 122) (end 103.75 122.05) (width 0.3) (layer "F.Cu") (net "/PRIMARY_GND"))
 (via (at 103.7 122) (size 0.6) (drill 0.3) (layers "F.Cu" "B.Cu") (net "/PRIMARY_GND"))
 (via (at 94 127.8) (size 0.6) (drill 0.3) (layers "F.Cu" "B.Cu") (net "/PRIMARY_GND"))
 (segment (start 103.7 123.4) (end 103.7 122) (width 0.3) (layer "B.Cu") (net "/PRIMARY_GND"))
 (segment (start 100.5 129) (end 100.5 126.6) (width 0.3) (layer "B.Cu") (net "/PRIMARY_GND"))
 (segment (start 103.7 123.4) (end 103.75 123.4) (width 0.3) (layer "B.Cu") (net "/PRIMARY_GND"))
 (segment (start 97.1 128.199999) (end 97.3 128.4) (width 0.3) (layer "B.Cu") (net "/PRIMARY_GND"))
 (segment (start 94 127.8) (end 95.3 127.8) (width 0.3) (layer "B.Cu") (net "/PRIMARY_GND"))
 (segment (start 95.7 128.199999) (end 97.1 128.199999) (width 0.3) (layer "B.Cu") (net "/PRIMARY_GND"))
 (segment (start 97.3 128.4) (end 97.5 128.4) (width 0.3) (layer "B.Cu") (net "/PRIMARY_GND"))
 (segment (start 97.5 128.4) (end 98.1 129) (width 0.3) (layer "B.Cu") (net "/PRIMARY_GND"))
 (segment (start 100.5 126.6) (end 103.7 123.4) (width 0.3) (layer "B.Cu") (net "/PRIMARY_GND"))
 (segment (start 103.75 123.4) (end 103.7 123.4) (width 0.3) (layer "B.Cu") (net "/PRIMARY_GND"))
 (segment (start 95.3 127.8) (end 95.7 128.199999) (width 0.3) (layer "B.Cu") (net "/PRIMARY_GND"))
 (segment (start 98.1 129) (end 100.5 129) (width 0.3) (layer "B.Cu") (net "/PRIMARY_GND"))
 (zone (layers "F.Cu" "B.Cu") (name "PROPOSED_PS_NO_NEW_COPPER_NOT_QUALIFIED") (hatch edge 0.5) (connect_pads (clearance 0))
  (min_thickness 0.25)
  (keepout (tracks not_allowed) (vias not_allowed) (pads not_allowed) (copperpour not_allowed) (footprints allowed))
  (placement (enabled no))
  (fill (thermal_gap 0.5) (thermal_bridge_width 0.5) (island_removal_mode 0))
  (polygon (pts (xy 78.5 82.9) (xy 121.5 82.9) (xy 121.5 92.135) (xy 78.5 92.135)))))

